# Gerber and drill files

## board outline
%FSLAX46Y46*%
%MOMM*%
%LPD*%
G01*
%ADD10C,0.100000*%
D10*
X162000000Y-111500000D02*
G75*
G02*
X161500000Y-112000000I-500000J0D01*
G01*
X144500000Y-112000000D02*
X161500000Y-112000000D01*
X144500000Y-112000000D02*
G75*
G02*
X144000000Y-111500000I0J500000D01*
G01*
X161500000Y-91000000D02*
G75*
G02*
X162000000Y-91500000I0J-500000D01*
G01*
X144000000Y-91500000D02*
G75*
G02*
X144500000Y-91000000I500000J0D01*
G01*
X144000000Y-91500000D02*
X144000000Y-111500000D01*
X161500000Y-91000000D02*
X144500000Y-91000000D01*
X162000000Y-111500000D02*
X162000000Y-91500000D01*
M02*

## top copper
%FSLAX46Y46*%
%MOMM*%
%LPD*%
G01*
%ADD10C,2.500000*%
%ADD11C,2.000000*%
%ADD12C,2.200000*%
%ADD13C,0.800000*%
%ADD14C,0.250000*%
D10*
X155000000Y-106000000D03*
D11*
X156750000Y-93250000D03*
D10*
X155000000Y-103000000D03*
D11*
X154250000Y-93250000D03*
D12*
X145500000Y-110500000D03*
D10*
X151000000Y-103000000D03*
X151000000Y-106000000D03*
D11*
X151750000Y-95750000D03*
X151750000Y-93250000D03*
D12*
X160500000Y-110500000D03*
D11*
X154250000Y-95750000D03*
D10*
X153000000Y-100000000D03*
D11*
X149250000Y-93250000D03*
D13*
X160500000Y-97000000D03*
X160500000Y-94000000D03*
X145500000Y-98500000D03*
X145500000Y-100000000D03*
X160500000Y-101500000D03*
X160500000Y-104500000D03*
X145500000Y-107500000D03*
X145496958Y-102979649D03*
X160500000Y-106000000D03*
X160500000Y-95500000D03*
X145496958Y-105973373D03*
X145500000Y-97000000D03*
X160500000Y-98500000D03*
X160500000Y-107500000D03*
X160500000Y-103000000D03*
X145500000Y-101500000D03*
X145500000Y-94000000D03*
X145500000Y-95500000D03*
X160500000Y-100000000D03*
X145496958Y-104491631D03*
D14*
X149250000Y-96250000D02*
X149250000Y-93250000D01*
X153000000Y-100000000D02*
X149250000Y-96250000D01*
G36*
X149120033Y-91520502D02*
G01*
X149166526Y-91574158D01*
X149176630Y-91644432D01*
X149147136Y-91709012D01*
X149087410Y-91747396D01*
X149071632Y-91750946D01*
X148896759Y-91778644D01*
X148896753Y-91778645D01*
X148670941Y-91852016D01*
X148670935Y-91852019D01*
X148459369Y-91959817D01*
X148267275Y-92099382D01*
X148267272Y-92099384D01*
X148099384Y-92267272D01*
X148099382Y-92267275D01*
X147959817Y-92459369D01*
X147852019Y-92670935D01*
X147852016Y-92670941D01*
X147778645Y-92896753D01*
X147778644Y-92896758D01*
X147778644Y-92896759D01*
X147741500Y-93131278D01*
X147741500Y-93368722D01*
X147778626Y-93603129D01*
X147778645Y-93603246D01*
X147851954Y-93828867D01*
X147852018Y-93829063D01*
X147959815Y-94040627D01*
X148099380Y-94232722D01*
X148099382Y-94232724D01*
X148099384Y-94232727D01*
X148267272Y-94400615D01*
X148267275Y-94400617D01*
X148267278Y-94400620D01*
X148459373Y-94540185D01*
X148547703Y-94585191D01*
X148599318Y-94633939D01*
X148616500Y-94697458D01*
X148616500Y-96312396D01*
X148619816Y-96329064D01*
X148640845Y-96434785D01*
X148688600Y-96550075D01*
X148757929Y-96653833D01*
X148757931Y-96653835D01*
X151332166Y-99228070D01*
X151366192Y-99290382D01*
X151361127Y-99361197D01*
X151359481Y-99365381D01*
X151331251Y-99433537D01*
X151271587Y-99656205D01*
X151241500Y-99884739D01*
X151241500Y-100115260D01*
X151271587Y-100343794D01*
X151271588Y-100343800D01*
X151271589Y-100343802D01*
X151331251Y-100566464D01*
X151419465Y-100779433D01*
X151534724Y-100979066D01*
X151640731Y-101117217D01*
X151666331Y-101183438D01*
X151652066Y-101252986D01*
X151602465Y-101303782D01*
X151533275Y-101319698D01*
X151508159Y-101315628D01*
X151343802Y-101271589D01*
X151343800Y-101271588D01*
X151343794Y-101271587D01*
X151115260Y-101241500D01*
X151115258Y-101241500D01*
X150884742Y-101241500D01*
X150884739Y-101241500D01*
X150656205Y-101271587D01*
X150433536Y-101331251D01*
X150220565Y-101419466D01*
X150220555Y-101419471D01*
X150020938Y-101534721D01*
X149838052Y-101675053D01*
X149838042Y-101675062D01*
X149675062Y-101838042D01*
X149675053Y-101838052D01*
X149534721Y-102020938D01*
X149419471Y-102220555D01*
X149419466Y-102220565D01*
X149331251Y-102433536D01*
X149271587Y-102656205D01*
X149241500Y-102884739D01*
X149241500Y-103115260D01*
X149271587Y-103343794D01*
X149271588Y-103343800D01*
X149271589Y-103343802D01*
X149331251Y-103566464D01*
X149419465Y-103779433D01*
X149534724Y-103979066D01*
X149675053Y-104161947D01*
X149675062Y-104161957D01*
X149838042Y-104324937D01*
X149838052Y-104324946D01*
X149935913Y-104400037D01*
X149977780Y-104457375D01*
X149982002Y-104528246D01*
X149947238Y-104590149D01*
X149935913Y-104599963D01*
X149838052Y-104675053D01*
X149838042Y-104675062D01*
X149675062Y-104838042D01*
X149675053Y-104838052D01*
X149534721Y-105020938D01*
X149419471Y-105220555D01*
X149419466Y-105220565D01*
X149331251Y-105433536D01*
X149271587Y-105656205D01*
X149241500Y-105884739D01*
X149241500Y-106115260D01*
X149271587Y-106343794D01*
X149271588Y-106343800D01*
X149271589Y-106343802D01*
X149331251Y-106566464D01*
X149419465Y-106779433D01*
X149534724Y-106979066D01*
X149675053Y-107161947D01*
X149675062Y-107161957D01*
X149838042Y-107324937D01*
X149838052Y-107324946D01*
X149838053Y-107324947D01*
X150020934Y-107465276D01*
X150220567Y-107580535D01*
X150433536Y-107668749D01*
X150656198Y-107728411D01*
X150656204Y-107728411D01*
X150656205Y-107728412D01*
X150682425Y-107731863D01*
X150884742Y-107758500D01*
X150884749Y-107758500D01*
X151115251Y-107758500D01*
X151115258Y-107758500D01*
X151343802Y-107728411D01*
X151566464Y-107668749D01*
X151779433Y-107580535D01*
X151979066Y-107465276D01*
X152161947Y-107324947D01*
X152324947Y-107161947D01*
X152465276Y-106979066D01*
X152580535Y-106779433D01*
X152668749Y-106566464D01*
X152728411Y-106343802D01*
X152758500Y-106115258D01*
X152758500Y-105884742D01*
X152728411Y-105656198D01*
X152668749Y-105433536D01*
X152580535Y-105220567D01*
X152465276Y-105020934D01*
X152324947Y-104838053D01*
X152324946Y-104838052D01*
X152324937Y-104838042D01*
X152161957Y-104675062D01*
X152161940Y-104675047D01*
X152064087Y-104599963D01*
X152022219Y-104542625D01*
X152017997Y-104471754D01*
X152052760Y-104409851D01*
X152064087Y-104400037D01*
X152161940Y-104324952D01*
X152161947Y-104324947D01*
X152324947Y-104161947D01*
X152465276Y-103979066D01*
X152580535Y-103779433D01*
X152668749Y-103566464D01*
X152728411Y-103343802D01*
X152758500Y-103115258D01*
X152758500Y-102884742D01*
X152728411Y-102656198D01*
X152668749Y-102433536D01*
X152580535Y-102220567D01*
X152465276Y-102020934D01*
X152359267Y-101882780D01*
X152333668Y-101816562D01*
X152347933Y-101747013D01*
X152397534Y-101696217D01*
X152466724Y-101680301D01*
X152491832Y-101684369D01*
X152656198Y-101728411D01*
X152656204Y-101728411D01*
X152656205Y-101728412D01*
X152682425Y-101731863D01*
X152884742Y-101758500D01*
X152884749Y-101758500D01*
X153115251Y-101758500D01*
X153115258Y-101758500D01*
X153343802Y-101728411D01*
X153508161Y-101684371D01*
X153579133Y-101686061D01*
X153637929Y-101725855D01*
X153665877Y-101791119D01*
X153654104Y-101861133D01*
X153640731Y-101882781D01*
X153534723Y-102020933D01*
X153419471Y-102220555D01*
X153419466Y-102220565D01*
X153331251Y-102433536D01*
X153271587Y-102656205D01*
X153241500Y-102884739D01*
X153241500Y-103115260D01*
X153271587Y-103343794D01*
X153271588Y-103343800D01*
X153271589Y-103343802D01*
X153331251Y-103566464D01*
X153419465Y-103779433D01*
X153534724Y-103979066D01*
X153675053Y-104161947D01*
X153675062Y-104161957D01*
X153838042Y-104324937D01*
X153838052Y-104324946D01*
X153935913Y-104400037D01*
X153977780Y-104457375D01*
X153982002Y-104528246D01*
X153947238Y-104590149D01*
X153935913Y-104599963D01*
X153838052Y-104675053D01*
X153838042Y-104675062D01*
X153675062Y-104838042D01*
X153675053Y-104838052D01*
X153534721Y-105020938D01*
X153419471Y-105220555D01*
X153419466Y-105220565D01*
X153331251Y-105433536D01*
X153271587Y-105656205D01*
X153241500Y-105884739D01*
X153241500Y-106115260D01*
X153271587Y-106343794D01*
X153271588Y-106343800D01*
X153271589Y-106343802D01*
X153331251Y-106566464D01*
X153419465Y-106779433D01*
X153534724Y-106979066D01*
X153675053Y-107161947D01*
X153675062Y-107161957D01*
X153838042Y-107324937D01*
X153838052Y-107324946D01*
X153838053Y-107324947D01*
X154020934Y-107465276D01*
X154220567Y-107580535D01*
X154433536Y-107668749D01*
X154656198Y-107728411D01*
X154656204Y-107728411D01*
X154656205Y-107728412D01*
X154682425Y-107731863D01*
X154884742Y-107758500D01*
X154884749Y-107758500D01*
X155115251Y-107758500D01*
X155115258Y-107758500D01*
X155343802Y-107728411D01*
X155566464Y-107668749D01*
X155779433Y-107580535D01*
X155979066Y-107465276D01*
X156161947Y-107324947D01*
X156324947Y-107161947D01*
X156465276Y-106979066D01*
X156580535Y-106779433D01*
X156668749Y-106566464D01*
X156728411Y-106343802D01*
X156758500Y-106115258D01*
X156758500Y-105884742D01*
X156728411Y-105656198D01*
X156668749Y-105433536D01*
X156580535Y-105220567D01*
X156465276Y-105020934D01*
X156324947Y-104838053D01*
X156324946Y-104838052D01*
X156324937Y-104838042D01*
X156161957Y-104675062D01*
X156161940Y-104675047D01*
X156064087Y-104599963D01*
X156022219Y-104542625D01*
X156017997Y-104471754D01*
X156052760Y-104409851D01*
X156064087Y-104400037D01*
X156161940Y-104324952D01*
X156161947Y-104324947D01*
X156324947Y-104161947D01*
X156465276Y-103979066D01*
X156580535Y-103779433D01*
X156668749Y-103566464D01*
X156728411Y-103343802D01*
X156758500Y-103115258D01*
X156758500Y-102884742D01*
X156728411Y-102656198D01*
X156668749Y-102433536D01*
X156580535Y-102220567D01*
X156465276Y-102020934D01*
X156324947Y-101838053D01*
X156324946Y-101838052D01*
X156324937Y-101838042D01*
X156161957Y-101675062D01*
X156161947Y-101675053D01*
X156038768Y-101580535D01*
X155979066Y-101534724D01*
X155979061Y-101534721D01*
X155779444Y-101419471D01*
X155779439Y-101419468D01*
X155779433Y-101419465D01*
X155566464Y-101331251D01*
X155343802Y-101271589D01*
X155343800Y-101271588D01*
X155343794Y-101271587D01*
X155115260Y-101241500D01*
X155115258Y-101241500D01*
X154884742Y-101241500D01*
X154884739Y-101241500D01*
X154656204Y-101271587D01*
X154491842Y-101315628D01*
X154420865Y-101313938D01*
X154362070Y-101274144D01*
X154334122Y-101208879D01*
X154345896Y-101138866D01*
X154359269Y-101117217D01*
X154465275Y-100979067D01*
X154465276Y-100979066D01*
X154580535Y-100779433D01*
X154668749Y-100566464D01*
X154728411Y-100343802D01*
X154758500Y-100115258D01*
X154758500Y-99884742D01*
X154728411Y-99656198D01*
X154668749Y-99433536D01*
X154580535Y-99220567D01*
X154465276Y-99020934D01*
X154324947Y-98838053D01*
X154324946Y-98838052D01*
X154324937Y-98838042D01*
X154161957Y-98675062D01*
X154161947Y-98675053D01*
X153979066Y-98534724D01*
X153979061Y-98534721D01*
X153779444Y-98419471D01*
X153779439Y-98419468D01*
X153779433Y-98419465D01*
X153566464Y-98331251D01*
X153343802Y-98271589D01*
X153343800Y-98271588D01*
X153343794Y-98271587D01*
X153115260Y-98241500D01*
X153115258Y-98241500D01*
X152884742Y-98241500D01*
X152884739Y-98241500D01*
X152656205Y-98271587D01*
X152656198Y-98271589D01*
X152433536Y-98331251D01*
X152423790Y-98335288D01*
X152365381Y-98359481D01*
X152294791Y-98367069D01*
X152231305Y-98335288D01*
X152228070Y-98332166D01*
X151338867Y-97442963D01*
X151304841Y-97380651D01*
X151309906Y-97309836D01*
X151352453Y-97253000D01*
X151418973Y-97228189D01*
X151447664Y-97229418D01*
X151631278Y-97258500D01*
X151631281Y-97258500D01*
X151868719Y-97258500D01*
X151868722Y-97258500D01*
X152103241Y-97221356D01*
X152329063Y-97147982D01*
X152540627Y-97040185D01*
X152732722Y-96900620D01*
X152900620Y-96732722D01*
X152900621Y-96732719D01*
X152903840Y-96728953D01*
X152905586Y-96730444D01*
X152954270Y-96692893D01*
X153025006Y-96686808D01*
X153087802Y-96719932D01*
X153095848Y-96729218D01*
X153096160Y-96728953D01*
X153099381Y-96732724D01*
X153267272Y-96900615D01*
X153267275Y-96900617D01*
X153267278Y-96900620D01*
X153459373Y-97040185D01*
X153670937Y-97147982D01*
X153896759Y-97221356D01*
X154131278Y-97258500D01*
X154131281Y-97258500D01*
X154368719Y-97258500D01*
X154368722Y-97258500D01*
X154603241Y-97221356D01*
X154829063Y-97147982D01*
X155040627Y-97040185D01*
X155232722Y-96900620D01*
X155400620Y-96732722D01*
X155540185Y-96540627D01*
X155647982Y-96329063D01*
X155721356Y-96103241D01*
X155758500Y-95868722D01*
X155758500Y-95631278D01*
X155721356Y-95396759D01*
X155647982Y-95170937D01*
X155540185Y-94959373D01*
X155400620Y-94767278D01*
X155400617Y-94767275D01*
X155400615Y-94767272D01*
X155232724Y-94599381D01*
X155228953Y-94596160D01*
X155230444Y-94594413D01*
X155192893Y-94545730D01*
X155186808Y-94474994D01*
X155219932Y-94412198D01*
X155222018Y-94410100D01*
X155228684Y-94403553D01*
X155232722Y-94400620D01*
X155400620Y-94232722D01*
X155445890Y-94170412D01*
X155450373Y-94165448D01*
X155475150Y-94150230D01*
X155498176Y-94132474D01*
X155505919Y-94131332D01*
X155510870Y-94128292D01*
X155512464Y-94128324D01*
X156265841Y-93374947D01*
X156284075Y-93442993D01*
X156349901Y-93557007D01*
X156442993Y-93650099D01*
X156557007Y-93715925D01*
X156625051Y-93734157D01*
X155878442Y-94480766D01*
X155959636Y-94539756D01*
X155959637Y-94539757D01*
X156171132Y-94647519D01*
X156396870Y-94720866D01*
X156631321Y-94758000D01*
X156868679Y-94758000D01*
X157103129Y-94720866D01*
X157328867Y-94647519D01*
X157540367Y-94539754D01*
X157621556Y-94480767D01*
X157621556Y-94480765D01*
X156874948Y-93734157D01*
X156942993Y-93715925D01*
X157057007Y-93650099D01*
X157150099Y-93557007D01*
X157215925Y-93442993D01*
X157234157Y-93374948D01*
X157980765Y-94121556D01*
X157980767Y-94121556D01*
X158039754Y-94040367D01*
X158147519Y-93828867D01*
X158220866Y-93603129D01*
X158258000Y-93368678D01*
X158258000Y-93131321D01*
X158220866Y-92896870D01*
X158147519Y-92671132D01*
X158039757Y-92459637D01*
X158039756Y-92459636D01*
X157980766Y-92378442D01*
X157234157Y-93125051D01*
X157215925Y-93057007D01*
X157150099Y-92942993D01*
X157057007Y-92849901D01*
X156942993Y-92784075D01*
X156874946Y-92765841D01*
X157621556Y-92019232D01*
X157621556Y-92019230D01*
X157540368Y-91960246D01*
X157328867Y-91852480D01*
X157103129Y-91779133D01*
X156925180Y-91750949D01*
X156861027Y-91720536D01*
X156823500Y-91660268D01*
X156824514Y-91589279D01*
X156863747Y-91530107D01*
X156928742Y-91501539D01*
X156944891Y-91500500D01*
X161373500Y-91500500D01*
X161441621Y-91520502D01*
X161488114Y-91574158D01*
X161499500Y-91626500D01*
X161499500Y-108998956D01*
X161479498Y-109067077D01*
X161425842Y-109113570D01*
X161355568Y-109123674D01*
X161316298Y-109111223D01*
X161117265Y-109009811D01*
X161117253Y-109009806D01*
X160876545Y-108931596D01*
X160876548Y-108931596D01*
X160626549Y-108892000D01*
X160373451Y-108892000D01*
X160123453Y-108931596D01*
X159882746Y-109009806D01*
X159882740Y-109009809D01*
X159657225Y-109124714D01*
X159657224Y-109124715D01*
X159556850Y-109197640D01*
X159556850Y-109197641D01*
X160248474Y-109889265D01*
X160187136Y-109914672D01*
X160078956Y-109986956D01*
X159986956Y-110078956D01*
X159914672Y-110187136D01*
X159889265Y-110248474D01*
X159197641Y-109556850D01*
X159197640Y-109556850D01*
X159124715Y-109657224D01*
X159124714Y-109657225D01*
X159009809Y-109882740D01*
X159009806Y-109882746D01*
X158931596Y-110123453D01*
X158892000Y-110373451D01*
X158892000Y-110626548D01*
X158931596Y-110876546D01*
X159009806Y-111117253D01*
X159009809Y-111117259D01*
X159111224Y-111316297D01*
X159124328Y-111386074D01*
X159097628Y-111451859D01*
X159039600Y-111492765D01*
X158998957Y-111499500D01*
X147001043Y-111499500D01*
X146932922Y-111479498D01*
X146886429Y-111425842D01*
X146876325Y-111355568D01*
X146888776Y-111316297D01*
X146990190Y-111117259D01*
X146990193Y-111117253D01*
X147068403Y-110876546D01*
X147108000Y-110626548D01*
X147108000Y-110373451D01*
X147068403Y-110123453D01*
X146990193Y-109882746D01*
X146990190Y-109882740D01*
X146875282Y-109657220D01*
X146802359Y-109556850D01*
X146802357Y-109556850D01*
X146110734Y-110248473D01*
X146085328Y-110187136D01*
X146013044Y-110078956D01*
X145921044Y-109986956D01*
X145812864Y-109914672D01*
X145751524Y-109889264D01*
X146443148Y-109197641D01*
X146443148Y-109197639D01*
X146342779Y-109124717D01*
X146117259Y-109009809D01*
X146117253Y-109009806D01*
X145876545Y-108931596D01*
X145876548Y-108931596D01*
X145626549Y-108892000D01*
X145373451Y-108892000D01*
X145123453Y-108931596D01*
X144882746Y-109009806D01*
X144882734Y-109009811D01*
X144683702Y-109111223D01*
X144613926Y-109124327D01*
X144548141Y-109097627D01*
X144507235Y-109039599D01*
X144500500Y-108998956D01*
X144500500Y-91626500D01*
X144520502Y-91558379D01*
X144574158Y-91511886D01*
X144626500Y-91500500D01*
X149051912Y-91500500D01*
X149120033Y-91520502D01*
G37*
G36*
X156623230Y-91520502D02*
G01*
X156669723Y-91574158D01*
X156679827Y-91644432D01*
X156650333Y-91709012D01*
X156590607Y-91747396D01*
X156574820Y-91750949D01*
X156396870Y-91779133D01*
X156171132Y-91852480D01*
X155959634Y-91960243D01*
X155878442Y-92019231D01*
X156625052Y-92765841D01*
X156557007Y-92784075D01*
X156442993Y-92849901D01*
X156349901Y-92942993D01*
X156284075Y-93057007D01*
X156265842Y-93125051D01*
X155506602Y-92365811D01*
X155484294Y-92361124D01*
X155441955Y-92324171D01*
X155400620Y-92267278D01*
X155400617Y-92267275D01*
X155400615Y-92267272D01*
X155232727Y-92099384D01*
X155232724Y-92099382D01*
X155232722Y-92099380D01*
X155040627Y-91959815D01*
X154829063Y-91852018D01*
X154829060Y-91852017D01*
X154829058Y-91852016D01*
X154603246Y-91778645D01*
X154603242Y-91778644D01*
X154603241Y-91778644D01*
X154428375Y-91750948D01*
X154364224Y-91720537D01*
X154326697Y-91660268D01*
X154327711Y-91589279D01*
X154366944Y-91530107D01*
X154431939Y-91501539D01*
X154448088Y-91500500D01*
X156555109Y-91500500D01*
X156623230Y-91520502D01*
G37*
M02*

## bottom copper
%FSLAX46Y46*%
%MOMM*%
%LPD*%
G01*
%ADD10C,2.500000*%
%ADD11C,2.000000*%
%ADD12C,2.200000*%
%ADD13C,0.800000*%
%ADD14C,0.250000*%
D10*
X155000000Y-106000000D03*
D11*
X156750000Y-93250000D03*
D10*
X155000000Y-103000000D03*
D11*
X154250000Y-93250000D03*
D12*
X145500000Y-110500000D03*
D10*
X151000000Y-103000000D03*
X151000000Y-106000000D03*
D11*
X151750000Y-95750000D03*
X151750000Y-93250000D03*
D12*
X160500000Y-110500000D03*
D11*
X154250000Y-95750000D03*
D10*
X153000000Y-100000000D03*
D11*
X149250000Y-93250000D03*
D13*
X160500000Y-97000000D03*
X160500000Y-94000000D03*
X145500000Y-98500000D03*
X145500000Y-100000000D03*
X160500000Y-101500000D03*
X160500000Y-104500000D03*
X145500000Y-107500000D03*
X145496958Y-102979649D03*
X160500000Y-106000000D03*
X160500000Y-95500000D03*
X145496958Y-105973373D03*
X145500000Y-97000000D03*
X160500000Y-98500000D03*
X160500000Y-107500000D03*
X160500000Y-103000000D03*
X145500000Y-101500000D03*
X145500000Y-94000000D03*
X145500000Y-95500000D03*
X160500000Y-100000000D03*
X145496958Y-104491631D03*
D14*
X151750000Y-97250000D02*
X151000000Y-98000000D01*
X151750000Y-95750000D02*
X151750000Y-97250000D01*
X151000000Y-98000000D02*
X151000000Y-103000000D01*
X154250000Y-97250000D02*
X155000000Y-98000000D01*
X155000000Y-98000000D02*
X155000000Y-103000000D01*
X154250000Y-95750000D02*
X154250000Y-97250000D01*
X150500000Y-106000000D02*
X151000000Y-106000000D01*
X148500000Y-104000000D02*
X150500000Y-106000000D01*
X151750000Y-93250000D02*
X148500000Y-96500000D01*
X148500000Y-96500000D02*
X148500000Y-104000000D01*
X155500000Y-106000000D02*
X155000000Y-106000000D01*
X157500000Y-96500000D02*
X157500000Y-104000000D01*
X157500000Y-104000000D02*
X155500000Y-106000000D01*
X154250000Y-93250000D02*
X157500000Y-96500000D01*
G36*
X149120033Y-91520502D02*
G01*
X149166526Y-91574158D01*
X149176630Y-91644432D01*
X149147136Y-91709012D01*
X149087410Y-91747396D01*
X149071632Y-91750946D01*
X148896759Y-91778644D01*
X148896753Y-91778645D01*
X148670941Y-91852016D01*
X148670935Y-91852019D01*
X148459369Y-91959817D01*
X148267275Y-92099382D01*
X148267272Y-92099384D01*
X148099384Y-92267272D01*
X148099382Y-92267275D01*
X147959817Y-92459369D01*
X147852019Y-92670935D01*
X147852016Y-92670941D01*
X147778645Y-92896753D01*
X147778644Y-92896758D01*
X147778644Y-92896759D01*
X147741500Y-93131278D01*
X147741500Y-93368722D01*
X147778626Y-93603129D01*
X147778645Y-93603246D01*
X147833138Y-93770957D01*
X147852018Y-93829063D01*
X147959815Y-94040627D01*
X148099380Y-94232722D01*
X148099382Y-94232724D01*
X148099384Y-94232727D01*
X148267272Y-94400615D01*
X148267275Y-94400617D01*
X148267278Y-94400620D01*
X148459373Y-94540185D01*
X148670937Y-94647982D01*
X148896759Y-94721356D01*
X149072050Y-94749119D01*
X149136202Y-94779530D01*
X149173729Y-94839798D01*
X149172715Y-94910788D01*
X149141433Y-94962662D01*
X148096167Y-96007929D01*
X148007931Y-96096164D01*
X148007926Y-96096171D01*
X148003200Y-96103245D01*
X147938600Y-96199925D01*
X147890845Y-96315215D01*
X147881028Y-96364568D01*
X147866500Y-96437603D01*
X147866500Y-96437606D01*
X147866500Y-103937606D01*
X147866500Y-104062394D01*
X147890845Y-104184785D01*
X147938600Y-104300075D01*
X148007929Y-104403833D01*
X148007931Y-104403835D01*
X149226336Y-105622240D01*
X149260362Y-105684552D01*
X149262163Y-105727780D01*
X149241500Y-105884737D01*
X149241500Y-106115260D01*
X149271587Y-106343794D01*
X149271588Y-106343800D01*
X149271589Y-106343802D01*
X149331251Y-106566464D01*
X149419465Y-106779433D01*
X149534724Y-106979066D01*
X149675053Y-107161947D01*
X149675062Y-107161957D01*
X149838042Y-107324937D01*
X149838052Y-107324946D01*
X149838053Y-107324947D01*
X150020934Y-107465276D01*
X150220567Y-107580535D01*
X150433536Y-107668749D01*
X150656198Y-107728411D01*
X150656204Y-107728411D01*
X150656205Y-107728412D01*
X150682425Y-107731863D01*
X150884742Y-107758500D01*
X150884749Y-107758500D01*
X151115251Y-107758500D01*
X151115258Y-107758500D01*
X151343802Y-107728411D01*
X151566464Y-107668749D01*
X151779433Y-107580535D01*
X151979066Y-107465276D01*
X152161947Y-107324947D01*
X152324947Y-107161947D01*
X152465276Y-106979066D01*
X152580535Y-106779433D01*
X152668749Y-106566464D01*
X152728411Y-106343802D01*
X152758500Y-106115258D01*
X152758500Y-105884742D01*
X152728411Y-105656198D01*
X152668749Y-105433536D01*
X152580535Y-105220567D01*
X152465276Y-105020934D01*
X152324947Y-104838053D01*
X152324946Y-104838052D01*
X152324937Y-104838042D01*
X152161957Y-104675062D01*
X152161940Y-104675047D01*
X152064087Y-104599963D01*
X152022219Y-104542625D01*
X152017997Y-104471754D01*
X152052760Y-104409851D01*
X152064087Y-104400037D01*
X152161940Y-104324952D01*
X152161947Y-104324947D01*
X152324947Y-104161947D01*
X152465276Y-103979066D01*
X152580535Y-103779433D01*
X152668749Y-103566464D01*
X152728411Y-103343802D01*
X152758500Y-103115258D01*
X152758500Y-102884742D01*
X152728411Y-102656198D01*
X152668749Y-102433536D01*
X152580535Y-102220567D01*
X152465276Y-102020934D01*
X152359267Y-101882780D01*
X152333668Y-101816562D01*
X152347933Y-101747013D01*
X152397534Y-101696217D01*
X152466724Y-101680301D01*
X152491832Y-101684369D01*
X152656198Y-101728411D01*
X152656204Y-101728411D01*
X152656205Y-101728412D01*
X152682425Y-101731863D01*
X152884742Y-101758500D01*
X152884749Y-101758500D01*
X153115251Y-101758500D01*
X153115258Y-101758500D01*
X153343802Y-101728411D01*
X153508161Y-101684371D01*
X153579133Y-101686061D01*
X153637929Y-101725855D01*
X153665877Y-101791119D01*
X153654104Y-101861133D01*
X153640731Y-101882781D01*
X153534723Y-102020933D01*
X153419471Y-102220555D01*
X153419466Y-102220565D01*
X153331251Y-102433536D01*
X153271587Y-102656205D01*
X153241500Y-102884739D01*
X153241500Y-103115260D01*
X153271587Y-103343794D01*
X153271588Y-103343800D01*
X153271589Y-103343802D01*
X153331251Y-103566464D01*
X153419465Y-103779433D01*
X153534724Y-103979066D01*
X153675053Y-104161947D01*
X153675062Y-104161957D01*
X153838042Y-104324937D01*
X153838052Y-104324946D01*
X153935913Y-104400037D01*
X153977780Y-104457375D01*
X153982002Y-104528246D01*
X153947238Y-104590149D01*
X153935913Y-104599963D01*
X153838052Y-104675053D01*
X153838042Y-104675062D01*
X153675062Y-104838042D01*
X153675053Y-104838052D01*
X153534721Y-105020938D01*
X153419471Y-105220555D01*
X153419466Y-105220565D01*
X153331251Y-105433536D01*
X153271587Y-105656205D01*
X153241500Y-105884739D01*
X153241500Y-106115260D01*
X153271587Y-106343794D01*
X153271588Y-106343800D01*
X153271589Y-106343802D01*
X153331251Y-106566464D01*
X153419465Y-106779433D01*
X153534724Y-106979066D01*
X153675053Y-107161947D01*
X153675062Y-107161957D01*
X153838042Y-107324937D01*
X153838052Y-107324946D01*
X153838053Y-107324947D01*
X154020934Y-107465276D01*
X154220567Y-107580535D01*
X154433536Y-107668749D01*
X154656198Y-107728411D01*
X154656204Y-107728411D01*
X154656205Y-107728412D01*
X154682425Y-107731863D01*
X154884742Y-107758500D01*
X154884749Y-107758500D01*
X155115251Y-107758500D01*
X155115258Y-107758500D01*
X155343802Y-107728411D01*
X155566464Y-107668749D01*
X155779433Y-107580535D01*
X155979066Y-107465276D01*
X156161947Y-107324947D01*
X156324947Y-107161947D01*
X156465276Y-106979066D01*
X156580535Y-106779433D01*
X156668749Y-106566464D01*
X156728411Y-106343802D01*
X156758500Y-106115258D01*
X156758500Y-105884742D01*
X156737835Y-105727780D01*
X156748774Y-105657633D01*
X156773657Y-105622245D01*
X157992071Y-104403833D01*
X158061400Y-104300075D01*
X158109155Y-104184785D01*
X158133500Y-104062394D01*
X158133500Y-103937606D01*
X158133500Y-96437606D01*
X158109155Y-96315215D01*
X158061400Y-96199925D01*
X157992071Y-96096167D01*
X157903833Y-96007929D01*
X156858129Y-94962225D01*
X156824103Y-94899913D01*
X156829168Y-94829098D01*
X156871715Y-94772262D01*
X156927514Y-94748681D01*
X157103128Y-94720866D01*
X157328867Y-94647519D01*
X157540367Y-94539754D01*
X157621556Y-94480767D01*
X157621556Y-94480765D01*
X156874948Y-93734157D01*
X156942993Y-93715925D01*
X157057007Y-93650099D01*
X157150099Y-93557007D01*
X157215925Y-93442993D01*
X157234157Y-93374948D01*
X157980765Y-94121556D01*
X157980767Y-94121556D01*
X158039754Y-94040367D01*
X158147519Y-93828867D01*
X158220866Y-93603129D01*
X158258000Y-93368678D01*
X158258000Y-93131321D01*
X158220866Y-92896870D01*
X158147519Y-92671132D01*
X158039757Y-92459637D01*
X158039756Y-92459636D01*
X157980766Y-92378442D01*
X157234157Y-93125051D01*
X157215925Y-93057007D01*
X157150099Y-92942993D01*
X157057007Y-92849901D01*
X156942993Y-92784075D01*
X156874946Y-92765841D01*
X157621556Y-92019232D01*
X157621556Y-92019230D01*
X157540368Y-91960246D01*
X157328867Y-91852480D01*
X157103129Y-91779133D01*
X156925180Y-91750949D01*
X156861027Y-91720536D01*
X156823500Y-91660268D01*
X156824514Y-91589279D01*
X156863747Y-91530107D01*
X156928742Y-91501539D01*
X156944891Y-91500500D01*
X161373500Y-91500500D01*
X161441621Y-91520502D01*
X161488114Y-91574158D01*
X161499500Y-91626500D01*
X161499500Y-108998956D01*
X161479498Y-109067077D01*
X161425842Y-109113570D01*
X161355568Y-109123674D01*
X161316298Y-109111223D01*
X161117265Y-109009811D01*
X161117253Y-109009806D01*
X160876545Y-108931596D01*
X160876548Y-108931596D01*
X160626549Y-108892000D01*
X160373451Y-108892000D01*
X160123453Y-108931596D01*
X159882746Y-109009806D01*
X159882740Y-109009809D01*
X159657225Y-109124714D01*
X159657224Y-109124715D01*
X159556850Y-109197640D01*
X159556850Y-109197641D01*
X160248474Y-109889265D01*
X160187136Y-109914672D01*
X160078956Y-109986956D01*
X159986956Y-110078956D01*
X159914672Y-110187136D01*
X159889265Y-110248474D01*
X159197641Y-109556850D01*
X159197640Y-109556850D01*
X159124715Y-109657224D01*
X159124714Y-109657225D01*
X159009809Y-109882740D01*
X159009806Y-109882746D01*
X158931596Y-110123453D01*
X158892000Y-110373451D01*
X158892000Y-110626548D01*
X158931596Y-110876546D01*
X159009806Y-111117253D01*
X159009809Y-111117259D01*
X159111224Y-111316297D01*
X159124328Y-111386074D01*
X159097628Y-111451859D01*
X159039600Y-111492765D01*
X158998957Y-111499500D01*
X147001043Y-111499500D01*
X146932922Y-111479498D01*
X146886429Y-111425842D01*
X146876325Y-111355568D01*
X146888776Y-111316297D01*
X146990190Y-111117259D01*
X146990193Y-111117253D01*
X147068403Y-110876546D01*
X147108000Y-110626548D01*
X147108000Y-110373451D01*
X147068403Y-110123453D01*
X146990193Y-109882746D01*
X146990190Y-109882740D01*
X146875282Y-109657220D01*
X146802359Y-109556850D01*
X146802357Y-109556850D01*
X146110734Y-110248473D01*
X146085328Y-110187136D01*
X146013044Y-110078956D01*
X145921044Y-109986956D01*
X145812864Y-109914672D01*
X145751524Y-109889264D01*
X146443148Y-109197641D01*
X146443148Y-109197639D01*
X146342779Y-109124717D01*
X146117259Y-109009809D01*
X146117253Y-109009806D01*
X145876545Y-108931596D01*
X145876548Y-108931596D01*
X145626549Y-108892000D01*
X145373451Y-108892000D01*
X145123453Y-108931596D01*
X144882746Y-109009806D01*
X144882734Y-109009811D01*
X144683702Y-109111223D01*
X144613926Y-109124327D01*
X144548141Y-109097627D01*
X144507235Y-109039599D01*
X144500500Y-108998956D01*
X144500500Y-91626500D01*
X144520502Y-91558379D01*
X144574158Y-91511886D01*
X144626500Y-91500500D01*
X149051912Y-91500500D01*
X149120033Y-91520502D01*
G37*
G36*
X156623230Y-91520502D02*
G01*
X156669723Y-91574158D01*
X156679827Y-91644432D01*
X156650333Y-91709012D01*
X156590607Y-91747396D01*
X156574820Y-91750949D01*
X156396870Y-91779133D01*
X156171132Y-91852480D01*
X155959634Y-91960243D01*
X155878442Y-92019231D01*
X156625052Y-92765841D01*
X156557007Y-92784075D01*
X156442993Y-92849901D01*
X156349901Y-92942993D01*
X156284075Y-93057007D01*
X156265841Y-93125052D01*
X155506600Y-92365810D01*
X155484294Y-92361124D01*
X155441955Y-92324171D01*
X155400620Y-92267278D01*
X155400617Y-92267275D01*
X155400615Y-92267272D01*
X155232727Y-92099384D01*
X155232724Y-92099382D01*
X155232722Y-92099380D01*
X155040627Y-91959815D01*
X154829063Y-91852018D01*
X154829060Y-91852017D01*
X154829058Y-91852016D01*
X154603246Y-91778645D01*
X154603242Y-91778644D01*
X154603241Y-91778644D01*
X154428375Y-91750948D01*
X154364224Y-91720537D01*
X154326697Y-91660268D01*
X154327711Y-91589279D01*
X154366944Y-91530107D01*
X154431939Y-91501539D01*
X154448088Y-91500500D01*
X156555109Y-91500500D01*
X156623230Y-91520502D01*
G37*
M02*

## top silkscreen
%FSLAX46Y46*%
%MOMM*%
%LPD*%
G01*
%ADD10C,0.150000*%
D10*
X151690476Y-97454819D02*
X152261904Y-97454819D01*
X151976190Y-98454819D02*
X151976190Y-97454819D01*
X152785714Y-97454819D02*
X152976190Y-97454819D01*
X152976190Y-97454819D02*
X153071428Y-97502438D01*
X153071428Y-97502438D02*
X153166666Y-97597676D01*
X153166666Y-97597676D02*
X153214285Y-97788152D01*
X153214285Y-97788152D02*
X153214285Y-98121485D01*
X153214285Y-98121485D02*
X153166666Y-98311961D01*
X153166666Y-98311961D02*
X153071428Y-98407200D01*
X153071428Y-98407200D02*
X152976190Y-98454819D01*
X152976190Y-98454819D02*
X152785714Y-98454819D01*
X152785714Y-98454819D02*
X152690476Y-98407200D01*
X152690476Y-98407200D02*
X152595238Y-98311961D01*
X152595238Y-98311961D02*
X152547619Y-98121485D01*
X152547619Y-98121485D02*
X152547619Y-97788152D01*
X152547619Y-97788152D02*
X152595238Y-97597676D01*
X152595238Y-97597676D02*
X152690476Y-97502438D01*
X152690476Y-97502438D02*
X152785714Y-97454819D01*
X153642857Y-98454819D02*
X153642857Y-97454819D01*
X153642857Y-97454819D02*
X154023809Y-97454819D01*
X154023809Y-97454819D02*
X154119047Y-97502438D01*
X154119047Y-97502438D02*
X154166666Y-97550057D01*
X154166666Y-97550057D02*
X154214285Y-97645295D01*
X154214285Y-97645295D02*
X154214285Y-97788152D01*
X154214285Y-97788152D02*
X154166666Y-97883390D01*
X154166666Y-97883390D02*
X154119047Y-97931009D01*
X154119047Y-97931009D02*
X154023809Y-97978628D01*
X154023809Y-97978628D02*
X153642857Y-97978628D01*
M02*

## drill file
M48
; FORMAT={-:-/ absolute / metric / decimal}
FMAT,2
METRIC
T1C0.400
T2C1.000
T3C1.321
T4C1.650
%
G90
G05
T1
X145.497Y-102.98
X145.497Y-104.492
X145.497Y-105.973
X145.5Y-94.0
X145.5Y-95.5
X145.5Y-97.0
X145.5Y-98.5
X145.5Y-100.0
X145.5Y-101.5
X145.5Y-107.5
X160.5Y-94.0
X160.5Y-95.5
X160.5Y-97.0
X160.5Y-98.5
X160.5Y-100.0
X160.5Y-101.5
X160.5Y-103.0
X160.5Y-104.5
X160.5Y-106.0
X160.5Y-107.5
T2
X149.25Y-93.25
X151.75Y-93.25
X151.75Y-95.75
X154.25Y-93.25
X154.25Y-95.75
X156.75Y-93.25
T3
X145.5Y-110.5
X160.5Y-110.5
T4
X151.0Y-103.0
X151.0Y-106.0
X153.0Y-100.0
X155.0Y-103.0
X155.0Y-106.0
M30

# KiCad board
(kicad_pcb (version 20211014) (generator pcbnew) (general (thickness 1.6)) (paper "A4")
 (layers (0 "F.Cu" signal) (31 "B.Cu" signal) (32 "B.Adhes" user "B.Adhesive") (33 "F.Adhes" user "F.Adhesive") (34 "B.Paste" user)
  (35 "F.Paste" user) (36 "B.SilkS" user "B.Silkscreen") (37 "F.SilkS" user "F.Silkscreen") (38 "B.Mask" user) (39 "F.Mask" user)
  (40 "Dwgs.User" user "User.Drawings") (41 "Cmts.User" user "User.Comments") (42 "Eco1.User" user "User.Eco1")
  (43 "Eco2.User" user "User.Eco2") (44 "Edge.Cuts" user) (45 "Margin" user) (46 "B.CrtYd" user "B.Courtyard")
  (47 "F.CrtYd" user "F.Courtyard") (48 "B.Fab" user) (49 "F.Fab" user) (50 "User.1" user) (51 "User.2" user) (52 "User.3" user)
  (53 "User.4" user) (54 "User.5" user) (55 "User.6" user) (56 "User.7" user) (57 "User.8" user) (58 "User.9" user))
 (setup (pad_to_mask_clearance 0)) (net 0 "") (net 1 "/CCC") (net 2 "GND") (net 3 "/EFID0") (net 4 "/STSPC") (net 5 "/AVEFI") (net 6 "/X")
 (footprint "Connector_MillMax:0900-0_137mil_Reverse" (layer "F.Cu") (at 155 106)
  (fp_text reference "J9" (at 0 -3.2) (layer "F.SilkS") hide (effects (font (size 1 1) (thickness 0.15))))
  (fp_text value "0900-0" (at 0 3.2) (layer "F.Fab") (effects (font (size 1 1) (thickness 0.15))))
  (pad "1" thru_hole circle (at 0 0) (size 2.5 2.5) (drill 1.65) (layers *.Cu *.Mask) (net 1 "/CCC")))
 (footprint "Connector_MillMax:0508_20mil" (layer "F.Cu") (at 156.75 93.25)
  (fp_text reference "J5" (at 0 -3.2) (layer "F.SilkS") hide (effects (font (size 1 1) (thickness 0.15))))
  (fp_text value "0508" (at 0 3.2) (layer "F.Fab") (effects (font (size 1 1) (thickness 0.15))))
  (pad "1" thru_hole circle (at 0 0) (size 2 2) (drill 1) (layers *.Cu *.Mask) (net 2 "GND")))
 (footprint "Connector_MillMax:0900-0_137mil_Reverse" (layer "F.Cu") (at 155 103)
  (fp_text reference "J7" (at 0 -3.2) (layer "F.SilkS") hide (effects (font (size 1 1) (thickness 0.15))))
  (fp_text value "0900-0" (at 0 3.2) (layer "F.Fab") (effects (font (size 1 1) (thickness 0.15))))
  (pad "1" thru_hole circle (at 0 0) (size 2.5 2.5) (drill 1.65) (layers *.Cu *.Mask) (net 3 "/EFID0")))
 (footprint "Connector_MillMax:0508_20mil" (layer "F.Cu") (at 154.25 93.25)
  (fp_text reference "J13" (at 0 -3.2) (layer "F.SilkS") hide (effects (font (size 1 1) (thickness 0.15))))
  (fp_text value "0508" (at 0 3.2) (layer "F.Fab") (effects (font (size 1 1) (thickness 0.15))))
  (pad "1" thru_hole circle (at 0 0) (size 2 2) (drill 1) (layers *.Cu *.Mask) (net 1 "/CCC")))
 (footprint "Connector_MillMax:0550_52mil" (layer "F.Cu") (at 145.5 110.5)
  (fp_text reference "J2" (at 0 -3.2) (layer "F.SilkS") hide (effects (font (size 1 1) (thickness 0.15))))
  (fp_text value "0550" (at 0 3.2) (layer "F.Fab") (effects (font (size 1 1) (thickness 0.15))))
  (pad "1" thru_hole circle (at 0 0) (size 2.2 2.2) (drill 1.321) (layers *.Cu *.Mask) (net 2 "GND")))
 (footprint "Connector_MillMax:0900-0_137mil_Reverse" (layer "F.Cu") (at 151 103)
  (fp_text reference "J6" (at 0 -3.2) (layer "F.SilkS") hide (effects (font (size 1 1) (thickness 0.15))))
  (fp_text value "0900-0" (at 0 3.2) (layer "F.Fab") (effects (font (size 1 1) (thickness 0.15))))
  (pad "1" thru_hole circle (at 0 0) (size 2.5 2.5) (drill 1.65) (layers *.Cu *.Mask) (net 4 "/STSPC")))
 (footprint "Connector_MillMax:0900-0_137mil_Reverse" (layer "F.Cu") (at 151 106)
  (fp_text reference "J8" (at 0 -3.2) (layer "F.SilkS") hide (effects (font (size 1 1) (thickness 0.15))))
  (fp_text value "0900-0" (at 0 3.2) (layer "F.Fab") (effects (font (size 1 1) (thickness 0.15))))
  (pad "1" thru_hole circle (at 0 0) (size 2.5 2.5) (drill 1.65) (layers *.Cu *.Mask) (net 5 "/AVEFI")))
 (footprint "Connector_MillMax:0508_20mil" (layer "F.Cu") (at 151.75 95.75)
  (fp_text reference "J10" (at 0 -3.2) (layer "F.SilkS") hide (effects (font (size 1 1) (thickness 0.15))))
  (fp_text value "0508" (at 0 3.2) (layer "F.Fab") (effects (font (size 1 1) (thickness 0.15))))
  (pad "1" thru_hole circle (at 0 0) (size 2 2) (drill 1) (layers *.Cu *.Mask) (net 4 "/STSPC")))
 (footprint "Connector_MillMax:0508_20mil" (layer "F.Cu") (at 151.75 93.25)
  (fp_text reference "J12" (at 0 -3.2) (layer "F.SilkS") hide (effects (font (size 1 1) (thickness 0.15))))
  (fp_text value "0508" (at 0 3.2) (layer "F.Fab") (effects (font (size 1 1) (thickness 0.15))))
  (pad "1" thru_hole circle (at 0 0) (size 2 2) (drill 1) (layers *.Cu *.Mask) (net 5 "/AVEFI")))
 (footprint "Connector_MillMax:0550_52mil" (layer "F.Cu") (at 160.5 110.5)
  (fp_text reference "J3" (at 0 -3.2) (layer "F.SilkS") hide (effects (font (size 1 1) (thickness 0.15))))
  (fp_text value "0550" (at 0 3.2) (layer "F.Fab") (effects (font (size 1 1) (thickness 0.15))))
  (pad "1" thru_hole circle (at 0 0) (size 2.2 2.2) (drill 1.321) (layers *.Cu *.Mask) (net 2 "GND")))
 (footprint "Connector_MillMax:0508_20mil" (layer "F.Cu") (at 154.25 95.75)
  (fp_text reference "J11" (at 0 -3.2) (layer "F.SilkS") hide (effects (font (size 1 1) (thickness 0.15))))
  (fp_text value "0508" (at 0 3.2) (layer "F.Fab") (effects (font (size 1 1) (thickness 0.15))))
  (pad "1" thru_hole circle (at 0 0) (size 2 2) (drill 1) (layers *.Cu *.Mask) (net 3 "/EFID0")))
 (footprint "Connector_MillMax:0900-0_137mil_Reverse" (layer "F.Cu") (at 153 100)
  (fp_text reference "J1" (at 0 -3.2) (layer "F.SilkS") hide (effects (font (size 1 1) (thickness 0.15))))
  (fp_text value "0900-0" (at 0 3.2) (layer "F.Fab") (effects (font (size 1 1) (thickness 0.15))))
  (pad "1" thru_hole circle (at 0 0) (size 2.5 2.5) (drill 1.65) (layers *.Cu *.Mask) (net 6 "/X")))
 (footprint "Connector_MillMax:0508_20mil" (layer "F.Cu") (at 149.25 93.25)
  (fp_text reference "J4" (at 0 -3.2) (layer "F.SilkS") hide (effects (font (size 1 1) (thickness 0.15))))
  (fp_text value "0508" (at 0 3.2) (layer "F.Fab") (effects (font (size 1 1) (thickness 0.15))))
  (pad "1" thru_hole circle (at 0 0) (size 2 2) (drill 1) (layers *.Cu *.Mask) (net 6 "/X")))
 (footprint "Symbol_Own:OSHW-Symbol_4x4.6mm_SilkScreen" (layer "B.Cu") (at 153.035 110.222797 180)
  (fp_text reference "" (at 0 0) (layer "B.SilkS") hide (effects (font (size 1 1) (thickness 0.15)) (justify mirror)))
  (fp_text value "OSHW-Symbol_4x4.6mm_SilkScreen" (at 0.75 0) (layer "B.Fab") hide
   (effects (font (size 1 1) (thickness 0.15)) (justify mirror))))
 (gr_arc (start 162 111.5) (mid 161.853553 111.853553) (end 161.5 112) (layer "Edge.Cuts") (width 0.1))
 (gr_line (start 144.5 112) (end 161.5 112) (layer "Edge.Cuts") (width 0.1))
 (gr_arc (start 144.5 112) (mid 144.146447 111.853553) (end 144 111.5) (layer "Edge.Cuts") (width 0.1))
 (gr_arc (start 161.5 91) (mid 161.853553 91.146447) (end 162 91.5) (layer "Edge.Cuts") (width 0.1))
 (gr_arc (start 144 91.5) (mid 144.146447 91.146447) (end 144.5 91) (layer "Edge.Cuts") (width 0.1))
 (gr_line (start 144 91.5) (end 144 111.5) (layer "Edge.Cuts") (width 0.1))
 (gr_line (start 161.5 91) (end 144.5 91) (layer "Edge.Cuts") (width 0.1))
 (gr_line (start 162 111.5) (end 162 91.5) (layer "Edge.Cuts") (width 0.1))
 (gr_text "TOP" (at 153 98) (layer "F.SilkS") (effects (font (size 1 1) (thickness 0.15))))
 (segment (start 149.25 96.25) (end 149.25 93.25) (width 0.25) (layer "F.Cu") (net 6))
 (segment (start 153 100) (end 149.25 96.25) (width 0.25) (layer "F.Cu") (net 6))
 (via (at 160.5 97) (size 0.8) (drill 0.4) (layers "F.Cu" "B.Cu") (free) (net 2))
 (via (at 160.5 94) (size 0.8) (drill 0.4) (layers "F.Cu" "B.Cu") (free) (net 2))
 (via (at 145.5 98.5) (size 0.8) (drill 0.4) (layers "F.Cu" "B.Cu") (free) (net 2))
 (via (at 145.5 100) (size 0.8) (drill 0.4) (layers "F.Cu" "B.Cu") (free) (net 2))
 (via (at 160.5 101.5) (size 0.8) (drill 0.4) (layers "F.Cu" "B.Cu") (free) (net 2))
 (via (at 160.5 104.5) (size 0.8) (drill 0.4) (layers "F.Cu" "B.Cu") (free) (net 2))
 (via (at 145.5 107.5) (size 0.8) (drill 0.4) (layers "F.Cu" "B.Cu") (free) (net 2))
 (via (at 145.496958 102.979649) (size 0.8) (drill 0.4) (layers "F.Cu" "B.Cu") (free) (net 2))
 (via (at 160.5 106) (size 0.8) (drill 0.4) (layers "F.Cu" "B.Cu") (free) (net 2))
 (via (at 160.5 95.5) (size 0.8) (drill 0.4) (layers "F.Cu" "B.Cu") (free) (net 2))
 (via (at 145.496958 105.973373) (size 0.8) (drill 0.4) (layers "F.Cu" "B.Cu") (free) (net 2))
 (via (at 145.5 97) (size 0.8) (drill 0.4) (layers "F.Cu" "B.Cu") (free) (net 2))
 (via (at 160.5 98.5) (size 0.8) (drill 0.4) (layers "F.Cu" "B.Cu") (free) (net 2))
 (via (at 160.5 107.5) (size 0.8) (drill 0.4) (layers "F.Cu" "B.Cu") (free) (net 2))
 (via (at 160.5 103) (size 0.8) (drill 0.4) (layers "F.Cu" "B.Cu") (free) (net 2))
 (via (at 145.5 101.5) (size 0.8) (drill 0.4) (layers "F.Cu" "B.Cu") (free) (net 2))
 (via (at 145.5 94) (size 0.8) (drill 0.4) (layers "F.Cu" "B.Cu") (free) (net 2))
 (via (at 145.5 95.5) (size 0.8) (drill 0.4) (layers "F.Cu" "B.Cu") (free) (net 2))
 (via (at 160.5 100) (size 0.8) (drill 0.4) (layers "F.Cu" "B.Cu") (free) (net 2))
 (via (at 145.496958 104.491631) (size 0.8) (drill 0.4) (layers "F.Cu" "B.Cu") (free) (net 2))
 (segment (start 151.75 97.25) (end 151 98) (width 0.25) (layer "B.Cu") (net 4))
 (segment (start 151.75 95.75) (end 151.75 97.25) (width 0.25) (layer "B.Cu") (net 4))
 (segment (start 151 98) (end 151 103) (width 0.25) (layer "B.Cu") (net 4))
 (segment (start 154.25 97.25) (end 155 98) (width 0.25) (layer "B.Cu") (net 3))
 (segment (start 155 98) (end 155 103) (width 0.25) (layer "B.Cu") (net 3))
 (segment (start 154.25 95.75) (end 154.25 97.25) (width 0.25) (layer "B.Cu") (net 3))
 (segment (start 150.5 106) (end 151 106) (width 0.25) (layer "B.Cu") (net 5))
 (segment (start 148.5 104) (end 150.5 106) (width 0.25) (layer "B.Cu") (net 5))
 (segment (start 151.75 93.25) (end 148.5 96.5) (width 0.25) (layer "B.Cu") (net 5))
 (segment (start 148.5 96.5) (end 148.5 104) (width 0.25) (layer "B.Cu") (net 5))
 (segment (start 155.5 106) (end 155 106) (width 0.25) (layer "B.Cu") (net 1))
 (segment (start 157.5 96.5) (end 157.5 104) (width 0.25) (layer "B.Cu") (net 1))
 (segment (start 157.5 104) (end 155.5 106) (width 0.25) (layer "B.Cu") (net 1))
 (segment (start 154.25 93.25) (end 157.5 96.5) (width 0.25) (layer "B.Cu") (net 1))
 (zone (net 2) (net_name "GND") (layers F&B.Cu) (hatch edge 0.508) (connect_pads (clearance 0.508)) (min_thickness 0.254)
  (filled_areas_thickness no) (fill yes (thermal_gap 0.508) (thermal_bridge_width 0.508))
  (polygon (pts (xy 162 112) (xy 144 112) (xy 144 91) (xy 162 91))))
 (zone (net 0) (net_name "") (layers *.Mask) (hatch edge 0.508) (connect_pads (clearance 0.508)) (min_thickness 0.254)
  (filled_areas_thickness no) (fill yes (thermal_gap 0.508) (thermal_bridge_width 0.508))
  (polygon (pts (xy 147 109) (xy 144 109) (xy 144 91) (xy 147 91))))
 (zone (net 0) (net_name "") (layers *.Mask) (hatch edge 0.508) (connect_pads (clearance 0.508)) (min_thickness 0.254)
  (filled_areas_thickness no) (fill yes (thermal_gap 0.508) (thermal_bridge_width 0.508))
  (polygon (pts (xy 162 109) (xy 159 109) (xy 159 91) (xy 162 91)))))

